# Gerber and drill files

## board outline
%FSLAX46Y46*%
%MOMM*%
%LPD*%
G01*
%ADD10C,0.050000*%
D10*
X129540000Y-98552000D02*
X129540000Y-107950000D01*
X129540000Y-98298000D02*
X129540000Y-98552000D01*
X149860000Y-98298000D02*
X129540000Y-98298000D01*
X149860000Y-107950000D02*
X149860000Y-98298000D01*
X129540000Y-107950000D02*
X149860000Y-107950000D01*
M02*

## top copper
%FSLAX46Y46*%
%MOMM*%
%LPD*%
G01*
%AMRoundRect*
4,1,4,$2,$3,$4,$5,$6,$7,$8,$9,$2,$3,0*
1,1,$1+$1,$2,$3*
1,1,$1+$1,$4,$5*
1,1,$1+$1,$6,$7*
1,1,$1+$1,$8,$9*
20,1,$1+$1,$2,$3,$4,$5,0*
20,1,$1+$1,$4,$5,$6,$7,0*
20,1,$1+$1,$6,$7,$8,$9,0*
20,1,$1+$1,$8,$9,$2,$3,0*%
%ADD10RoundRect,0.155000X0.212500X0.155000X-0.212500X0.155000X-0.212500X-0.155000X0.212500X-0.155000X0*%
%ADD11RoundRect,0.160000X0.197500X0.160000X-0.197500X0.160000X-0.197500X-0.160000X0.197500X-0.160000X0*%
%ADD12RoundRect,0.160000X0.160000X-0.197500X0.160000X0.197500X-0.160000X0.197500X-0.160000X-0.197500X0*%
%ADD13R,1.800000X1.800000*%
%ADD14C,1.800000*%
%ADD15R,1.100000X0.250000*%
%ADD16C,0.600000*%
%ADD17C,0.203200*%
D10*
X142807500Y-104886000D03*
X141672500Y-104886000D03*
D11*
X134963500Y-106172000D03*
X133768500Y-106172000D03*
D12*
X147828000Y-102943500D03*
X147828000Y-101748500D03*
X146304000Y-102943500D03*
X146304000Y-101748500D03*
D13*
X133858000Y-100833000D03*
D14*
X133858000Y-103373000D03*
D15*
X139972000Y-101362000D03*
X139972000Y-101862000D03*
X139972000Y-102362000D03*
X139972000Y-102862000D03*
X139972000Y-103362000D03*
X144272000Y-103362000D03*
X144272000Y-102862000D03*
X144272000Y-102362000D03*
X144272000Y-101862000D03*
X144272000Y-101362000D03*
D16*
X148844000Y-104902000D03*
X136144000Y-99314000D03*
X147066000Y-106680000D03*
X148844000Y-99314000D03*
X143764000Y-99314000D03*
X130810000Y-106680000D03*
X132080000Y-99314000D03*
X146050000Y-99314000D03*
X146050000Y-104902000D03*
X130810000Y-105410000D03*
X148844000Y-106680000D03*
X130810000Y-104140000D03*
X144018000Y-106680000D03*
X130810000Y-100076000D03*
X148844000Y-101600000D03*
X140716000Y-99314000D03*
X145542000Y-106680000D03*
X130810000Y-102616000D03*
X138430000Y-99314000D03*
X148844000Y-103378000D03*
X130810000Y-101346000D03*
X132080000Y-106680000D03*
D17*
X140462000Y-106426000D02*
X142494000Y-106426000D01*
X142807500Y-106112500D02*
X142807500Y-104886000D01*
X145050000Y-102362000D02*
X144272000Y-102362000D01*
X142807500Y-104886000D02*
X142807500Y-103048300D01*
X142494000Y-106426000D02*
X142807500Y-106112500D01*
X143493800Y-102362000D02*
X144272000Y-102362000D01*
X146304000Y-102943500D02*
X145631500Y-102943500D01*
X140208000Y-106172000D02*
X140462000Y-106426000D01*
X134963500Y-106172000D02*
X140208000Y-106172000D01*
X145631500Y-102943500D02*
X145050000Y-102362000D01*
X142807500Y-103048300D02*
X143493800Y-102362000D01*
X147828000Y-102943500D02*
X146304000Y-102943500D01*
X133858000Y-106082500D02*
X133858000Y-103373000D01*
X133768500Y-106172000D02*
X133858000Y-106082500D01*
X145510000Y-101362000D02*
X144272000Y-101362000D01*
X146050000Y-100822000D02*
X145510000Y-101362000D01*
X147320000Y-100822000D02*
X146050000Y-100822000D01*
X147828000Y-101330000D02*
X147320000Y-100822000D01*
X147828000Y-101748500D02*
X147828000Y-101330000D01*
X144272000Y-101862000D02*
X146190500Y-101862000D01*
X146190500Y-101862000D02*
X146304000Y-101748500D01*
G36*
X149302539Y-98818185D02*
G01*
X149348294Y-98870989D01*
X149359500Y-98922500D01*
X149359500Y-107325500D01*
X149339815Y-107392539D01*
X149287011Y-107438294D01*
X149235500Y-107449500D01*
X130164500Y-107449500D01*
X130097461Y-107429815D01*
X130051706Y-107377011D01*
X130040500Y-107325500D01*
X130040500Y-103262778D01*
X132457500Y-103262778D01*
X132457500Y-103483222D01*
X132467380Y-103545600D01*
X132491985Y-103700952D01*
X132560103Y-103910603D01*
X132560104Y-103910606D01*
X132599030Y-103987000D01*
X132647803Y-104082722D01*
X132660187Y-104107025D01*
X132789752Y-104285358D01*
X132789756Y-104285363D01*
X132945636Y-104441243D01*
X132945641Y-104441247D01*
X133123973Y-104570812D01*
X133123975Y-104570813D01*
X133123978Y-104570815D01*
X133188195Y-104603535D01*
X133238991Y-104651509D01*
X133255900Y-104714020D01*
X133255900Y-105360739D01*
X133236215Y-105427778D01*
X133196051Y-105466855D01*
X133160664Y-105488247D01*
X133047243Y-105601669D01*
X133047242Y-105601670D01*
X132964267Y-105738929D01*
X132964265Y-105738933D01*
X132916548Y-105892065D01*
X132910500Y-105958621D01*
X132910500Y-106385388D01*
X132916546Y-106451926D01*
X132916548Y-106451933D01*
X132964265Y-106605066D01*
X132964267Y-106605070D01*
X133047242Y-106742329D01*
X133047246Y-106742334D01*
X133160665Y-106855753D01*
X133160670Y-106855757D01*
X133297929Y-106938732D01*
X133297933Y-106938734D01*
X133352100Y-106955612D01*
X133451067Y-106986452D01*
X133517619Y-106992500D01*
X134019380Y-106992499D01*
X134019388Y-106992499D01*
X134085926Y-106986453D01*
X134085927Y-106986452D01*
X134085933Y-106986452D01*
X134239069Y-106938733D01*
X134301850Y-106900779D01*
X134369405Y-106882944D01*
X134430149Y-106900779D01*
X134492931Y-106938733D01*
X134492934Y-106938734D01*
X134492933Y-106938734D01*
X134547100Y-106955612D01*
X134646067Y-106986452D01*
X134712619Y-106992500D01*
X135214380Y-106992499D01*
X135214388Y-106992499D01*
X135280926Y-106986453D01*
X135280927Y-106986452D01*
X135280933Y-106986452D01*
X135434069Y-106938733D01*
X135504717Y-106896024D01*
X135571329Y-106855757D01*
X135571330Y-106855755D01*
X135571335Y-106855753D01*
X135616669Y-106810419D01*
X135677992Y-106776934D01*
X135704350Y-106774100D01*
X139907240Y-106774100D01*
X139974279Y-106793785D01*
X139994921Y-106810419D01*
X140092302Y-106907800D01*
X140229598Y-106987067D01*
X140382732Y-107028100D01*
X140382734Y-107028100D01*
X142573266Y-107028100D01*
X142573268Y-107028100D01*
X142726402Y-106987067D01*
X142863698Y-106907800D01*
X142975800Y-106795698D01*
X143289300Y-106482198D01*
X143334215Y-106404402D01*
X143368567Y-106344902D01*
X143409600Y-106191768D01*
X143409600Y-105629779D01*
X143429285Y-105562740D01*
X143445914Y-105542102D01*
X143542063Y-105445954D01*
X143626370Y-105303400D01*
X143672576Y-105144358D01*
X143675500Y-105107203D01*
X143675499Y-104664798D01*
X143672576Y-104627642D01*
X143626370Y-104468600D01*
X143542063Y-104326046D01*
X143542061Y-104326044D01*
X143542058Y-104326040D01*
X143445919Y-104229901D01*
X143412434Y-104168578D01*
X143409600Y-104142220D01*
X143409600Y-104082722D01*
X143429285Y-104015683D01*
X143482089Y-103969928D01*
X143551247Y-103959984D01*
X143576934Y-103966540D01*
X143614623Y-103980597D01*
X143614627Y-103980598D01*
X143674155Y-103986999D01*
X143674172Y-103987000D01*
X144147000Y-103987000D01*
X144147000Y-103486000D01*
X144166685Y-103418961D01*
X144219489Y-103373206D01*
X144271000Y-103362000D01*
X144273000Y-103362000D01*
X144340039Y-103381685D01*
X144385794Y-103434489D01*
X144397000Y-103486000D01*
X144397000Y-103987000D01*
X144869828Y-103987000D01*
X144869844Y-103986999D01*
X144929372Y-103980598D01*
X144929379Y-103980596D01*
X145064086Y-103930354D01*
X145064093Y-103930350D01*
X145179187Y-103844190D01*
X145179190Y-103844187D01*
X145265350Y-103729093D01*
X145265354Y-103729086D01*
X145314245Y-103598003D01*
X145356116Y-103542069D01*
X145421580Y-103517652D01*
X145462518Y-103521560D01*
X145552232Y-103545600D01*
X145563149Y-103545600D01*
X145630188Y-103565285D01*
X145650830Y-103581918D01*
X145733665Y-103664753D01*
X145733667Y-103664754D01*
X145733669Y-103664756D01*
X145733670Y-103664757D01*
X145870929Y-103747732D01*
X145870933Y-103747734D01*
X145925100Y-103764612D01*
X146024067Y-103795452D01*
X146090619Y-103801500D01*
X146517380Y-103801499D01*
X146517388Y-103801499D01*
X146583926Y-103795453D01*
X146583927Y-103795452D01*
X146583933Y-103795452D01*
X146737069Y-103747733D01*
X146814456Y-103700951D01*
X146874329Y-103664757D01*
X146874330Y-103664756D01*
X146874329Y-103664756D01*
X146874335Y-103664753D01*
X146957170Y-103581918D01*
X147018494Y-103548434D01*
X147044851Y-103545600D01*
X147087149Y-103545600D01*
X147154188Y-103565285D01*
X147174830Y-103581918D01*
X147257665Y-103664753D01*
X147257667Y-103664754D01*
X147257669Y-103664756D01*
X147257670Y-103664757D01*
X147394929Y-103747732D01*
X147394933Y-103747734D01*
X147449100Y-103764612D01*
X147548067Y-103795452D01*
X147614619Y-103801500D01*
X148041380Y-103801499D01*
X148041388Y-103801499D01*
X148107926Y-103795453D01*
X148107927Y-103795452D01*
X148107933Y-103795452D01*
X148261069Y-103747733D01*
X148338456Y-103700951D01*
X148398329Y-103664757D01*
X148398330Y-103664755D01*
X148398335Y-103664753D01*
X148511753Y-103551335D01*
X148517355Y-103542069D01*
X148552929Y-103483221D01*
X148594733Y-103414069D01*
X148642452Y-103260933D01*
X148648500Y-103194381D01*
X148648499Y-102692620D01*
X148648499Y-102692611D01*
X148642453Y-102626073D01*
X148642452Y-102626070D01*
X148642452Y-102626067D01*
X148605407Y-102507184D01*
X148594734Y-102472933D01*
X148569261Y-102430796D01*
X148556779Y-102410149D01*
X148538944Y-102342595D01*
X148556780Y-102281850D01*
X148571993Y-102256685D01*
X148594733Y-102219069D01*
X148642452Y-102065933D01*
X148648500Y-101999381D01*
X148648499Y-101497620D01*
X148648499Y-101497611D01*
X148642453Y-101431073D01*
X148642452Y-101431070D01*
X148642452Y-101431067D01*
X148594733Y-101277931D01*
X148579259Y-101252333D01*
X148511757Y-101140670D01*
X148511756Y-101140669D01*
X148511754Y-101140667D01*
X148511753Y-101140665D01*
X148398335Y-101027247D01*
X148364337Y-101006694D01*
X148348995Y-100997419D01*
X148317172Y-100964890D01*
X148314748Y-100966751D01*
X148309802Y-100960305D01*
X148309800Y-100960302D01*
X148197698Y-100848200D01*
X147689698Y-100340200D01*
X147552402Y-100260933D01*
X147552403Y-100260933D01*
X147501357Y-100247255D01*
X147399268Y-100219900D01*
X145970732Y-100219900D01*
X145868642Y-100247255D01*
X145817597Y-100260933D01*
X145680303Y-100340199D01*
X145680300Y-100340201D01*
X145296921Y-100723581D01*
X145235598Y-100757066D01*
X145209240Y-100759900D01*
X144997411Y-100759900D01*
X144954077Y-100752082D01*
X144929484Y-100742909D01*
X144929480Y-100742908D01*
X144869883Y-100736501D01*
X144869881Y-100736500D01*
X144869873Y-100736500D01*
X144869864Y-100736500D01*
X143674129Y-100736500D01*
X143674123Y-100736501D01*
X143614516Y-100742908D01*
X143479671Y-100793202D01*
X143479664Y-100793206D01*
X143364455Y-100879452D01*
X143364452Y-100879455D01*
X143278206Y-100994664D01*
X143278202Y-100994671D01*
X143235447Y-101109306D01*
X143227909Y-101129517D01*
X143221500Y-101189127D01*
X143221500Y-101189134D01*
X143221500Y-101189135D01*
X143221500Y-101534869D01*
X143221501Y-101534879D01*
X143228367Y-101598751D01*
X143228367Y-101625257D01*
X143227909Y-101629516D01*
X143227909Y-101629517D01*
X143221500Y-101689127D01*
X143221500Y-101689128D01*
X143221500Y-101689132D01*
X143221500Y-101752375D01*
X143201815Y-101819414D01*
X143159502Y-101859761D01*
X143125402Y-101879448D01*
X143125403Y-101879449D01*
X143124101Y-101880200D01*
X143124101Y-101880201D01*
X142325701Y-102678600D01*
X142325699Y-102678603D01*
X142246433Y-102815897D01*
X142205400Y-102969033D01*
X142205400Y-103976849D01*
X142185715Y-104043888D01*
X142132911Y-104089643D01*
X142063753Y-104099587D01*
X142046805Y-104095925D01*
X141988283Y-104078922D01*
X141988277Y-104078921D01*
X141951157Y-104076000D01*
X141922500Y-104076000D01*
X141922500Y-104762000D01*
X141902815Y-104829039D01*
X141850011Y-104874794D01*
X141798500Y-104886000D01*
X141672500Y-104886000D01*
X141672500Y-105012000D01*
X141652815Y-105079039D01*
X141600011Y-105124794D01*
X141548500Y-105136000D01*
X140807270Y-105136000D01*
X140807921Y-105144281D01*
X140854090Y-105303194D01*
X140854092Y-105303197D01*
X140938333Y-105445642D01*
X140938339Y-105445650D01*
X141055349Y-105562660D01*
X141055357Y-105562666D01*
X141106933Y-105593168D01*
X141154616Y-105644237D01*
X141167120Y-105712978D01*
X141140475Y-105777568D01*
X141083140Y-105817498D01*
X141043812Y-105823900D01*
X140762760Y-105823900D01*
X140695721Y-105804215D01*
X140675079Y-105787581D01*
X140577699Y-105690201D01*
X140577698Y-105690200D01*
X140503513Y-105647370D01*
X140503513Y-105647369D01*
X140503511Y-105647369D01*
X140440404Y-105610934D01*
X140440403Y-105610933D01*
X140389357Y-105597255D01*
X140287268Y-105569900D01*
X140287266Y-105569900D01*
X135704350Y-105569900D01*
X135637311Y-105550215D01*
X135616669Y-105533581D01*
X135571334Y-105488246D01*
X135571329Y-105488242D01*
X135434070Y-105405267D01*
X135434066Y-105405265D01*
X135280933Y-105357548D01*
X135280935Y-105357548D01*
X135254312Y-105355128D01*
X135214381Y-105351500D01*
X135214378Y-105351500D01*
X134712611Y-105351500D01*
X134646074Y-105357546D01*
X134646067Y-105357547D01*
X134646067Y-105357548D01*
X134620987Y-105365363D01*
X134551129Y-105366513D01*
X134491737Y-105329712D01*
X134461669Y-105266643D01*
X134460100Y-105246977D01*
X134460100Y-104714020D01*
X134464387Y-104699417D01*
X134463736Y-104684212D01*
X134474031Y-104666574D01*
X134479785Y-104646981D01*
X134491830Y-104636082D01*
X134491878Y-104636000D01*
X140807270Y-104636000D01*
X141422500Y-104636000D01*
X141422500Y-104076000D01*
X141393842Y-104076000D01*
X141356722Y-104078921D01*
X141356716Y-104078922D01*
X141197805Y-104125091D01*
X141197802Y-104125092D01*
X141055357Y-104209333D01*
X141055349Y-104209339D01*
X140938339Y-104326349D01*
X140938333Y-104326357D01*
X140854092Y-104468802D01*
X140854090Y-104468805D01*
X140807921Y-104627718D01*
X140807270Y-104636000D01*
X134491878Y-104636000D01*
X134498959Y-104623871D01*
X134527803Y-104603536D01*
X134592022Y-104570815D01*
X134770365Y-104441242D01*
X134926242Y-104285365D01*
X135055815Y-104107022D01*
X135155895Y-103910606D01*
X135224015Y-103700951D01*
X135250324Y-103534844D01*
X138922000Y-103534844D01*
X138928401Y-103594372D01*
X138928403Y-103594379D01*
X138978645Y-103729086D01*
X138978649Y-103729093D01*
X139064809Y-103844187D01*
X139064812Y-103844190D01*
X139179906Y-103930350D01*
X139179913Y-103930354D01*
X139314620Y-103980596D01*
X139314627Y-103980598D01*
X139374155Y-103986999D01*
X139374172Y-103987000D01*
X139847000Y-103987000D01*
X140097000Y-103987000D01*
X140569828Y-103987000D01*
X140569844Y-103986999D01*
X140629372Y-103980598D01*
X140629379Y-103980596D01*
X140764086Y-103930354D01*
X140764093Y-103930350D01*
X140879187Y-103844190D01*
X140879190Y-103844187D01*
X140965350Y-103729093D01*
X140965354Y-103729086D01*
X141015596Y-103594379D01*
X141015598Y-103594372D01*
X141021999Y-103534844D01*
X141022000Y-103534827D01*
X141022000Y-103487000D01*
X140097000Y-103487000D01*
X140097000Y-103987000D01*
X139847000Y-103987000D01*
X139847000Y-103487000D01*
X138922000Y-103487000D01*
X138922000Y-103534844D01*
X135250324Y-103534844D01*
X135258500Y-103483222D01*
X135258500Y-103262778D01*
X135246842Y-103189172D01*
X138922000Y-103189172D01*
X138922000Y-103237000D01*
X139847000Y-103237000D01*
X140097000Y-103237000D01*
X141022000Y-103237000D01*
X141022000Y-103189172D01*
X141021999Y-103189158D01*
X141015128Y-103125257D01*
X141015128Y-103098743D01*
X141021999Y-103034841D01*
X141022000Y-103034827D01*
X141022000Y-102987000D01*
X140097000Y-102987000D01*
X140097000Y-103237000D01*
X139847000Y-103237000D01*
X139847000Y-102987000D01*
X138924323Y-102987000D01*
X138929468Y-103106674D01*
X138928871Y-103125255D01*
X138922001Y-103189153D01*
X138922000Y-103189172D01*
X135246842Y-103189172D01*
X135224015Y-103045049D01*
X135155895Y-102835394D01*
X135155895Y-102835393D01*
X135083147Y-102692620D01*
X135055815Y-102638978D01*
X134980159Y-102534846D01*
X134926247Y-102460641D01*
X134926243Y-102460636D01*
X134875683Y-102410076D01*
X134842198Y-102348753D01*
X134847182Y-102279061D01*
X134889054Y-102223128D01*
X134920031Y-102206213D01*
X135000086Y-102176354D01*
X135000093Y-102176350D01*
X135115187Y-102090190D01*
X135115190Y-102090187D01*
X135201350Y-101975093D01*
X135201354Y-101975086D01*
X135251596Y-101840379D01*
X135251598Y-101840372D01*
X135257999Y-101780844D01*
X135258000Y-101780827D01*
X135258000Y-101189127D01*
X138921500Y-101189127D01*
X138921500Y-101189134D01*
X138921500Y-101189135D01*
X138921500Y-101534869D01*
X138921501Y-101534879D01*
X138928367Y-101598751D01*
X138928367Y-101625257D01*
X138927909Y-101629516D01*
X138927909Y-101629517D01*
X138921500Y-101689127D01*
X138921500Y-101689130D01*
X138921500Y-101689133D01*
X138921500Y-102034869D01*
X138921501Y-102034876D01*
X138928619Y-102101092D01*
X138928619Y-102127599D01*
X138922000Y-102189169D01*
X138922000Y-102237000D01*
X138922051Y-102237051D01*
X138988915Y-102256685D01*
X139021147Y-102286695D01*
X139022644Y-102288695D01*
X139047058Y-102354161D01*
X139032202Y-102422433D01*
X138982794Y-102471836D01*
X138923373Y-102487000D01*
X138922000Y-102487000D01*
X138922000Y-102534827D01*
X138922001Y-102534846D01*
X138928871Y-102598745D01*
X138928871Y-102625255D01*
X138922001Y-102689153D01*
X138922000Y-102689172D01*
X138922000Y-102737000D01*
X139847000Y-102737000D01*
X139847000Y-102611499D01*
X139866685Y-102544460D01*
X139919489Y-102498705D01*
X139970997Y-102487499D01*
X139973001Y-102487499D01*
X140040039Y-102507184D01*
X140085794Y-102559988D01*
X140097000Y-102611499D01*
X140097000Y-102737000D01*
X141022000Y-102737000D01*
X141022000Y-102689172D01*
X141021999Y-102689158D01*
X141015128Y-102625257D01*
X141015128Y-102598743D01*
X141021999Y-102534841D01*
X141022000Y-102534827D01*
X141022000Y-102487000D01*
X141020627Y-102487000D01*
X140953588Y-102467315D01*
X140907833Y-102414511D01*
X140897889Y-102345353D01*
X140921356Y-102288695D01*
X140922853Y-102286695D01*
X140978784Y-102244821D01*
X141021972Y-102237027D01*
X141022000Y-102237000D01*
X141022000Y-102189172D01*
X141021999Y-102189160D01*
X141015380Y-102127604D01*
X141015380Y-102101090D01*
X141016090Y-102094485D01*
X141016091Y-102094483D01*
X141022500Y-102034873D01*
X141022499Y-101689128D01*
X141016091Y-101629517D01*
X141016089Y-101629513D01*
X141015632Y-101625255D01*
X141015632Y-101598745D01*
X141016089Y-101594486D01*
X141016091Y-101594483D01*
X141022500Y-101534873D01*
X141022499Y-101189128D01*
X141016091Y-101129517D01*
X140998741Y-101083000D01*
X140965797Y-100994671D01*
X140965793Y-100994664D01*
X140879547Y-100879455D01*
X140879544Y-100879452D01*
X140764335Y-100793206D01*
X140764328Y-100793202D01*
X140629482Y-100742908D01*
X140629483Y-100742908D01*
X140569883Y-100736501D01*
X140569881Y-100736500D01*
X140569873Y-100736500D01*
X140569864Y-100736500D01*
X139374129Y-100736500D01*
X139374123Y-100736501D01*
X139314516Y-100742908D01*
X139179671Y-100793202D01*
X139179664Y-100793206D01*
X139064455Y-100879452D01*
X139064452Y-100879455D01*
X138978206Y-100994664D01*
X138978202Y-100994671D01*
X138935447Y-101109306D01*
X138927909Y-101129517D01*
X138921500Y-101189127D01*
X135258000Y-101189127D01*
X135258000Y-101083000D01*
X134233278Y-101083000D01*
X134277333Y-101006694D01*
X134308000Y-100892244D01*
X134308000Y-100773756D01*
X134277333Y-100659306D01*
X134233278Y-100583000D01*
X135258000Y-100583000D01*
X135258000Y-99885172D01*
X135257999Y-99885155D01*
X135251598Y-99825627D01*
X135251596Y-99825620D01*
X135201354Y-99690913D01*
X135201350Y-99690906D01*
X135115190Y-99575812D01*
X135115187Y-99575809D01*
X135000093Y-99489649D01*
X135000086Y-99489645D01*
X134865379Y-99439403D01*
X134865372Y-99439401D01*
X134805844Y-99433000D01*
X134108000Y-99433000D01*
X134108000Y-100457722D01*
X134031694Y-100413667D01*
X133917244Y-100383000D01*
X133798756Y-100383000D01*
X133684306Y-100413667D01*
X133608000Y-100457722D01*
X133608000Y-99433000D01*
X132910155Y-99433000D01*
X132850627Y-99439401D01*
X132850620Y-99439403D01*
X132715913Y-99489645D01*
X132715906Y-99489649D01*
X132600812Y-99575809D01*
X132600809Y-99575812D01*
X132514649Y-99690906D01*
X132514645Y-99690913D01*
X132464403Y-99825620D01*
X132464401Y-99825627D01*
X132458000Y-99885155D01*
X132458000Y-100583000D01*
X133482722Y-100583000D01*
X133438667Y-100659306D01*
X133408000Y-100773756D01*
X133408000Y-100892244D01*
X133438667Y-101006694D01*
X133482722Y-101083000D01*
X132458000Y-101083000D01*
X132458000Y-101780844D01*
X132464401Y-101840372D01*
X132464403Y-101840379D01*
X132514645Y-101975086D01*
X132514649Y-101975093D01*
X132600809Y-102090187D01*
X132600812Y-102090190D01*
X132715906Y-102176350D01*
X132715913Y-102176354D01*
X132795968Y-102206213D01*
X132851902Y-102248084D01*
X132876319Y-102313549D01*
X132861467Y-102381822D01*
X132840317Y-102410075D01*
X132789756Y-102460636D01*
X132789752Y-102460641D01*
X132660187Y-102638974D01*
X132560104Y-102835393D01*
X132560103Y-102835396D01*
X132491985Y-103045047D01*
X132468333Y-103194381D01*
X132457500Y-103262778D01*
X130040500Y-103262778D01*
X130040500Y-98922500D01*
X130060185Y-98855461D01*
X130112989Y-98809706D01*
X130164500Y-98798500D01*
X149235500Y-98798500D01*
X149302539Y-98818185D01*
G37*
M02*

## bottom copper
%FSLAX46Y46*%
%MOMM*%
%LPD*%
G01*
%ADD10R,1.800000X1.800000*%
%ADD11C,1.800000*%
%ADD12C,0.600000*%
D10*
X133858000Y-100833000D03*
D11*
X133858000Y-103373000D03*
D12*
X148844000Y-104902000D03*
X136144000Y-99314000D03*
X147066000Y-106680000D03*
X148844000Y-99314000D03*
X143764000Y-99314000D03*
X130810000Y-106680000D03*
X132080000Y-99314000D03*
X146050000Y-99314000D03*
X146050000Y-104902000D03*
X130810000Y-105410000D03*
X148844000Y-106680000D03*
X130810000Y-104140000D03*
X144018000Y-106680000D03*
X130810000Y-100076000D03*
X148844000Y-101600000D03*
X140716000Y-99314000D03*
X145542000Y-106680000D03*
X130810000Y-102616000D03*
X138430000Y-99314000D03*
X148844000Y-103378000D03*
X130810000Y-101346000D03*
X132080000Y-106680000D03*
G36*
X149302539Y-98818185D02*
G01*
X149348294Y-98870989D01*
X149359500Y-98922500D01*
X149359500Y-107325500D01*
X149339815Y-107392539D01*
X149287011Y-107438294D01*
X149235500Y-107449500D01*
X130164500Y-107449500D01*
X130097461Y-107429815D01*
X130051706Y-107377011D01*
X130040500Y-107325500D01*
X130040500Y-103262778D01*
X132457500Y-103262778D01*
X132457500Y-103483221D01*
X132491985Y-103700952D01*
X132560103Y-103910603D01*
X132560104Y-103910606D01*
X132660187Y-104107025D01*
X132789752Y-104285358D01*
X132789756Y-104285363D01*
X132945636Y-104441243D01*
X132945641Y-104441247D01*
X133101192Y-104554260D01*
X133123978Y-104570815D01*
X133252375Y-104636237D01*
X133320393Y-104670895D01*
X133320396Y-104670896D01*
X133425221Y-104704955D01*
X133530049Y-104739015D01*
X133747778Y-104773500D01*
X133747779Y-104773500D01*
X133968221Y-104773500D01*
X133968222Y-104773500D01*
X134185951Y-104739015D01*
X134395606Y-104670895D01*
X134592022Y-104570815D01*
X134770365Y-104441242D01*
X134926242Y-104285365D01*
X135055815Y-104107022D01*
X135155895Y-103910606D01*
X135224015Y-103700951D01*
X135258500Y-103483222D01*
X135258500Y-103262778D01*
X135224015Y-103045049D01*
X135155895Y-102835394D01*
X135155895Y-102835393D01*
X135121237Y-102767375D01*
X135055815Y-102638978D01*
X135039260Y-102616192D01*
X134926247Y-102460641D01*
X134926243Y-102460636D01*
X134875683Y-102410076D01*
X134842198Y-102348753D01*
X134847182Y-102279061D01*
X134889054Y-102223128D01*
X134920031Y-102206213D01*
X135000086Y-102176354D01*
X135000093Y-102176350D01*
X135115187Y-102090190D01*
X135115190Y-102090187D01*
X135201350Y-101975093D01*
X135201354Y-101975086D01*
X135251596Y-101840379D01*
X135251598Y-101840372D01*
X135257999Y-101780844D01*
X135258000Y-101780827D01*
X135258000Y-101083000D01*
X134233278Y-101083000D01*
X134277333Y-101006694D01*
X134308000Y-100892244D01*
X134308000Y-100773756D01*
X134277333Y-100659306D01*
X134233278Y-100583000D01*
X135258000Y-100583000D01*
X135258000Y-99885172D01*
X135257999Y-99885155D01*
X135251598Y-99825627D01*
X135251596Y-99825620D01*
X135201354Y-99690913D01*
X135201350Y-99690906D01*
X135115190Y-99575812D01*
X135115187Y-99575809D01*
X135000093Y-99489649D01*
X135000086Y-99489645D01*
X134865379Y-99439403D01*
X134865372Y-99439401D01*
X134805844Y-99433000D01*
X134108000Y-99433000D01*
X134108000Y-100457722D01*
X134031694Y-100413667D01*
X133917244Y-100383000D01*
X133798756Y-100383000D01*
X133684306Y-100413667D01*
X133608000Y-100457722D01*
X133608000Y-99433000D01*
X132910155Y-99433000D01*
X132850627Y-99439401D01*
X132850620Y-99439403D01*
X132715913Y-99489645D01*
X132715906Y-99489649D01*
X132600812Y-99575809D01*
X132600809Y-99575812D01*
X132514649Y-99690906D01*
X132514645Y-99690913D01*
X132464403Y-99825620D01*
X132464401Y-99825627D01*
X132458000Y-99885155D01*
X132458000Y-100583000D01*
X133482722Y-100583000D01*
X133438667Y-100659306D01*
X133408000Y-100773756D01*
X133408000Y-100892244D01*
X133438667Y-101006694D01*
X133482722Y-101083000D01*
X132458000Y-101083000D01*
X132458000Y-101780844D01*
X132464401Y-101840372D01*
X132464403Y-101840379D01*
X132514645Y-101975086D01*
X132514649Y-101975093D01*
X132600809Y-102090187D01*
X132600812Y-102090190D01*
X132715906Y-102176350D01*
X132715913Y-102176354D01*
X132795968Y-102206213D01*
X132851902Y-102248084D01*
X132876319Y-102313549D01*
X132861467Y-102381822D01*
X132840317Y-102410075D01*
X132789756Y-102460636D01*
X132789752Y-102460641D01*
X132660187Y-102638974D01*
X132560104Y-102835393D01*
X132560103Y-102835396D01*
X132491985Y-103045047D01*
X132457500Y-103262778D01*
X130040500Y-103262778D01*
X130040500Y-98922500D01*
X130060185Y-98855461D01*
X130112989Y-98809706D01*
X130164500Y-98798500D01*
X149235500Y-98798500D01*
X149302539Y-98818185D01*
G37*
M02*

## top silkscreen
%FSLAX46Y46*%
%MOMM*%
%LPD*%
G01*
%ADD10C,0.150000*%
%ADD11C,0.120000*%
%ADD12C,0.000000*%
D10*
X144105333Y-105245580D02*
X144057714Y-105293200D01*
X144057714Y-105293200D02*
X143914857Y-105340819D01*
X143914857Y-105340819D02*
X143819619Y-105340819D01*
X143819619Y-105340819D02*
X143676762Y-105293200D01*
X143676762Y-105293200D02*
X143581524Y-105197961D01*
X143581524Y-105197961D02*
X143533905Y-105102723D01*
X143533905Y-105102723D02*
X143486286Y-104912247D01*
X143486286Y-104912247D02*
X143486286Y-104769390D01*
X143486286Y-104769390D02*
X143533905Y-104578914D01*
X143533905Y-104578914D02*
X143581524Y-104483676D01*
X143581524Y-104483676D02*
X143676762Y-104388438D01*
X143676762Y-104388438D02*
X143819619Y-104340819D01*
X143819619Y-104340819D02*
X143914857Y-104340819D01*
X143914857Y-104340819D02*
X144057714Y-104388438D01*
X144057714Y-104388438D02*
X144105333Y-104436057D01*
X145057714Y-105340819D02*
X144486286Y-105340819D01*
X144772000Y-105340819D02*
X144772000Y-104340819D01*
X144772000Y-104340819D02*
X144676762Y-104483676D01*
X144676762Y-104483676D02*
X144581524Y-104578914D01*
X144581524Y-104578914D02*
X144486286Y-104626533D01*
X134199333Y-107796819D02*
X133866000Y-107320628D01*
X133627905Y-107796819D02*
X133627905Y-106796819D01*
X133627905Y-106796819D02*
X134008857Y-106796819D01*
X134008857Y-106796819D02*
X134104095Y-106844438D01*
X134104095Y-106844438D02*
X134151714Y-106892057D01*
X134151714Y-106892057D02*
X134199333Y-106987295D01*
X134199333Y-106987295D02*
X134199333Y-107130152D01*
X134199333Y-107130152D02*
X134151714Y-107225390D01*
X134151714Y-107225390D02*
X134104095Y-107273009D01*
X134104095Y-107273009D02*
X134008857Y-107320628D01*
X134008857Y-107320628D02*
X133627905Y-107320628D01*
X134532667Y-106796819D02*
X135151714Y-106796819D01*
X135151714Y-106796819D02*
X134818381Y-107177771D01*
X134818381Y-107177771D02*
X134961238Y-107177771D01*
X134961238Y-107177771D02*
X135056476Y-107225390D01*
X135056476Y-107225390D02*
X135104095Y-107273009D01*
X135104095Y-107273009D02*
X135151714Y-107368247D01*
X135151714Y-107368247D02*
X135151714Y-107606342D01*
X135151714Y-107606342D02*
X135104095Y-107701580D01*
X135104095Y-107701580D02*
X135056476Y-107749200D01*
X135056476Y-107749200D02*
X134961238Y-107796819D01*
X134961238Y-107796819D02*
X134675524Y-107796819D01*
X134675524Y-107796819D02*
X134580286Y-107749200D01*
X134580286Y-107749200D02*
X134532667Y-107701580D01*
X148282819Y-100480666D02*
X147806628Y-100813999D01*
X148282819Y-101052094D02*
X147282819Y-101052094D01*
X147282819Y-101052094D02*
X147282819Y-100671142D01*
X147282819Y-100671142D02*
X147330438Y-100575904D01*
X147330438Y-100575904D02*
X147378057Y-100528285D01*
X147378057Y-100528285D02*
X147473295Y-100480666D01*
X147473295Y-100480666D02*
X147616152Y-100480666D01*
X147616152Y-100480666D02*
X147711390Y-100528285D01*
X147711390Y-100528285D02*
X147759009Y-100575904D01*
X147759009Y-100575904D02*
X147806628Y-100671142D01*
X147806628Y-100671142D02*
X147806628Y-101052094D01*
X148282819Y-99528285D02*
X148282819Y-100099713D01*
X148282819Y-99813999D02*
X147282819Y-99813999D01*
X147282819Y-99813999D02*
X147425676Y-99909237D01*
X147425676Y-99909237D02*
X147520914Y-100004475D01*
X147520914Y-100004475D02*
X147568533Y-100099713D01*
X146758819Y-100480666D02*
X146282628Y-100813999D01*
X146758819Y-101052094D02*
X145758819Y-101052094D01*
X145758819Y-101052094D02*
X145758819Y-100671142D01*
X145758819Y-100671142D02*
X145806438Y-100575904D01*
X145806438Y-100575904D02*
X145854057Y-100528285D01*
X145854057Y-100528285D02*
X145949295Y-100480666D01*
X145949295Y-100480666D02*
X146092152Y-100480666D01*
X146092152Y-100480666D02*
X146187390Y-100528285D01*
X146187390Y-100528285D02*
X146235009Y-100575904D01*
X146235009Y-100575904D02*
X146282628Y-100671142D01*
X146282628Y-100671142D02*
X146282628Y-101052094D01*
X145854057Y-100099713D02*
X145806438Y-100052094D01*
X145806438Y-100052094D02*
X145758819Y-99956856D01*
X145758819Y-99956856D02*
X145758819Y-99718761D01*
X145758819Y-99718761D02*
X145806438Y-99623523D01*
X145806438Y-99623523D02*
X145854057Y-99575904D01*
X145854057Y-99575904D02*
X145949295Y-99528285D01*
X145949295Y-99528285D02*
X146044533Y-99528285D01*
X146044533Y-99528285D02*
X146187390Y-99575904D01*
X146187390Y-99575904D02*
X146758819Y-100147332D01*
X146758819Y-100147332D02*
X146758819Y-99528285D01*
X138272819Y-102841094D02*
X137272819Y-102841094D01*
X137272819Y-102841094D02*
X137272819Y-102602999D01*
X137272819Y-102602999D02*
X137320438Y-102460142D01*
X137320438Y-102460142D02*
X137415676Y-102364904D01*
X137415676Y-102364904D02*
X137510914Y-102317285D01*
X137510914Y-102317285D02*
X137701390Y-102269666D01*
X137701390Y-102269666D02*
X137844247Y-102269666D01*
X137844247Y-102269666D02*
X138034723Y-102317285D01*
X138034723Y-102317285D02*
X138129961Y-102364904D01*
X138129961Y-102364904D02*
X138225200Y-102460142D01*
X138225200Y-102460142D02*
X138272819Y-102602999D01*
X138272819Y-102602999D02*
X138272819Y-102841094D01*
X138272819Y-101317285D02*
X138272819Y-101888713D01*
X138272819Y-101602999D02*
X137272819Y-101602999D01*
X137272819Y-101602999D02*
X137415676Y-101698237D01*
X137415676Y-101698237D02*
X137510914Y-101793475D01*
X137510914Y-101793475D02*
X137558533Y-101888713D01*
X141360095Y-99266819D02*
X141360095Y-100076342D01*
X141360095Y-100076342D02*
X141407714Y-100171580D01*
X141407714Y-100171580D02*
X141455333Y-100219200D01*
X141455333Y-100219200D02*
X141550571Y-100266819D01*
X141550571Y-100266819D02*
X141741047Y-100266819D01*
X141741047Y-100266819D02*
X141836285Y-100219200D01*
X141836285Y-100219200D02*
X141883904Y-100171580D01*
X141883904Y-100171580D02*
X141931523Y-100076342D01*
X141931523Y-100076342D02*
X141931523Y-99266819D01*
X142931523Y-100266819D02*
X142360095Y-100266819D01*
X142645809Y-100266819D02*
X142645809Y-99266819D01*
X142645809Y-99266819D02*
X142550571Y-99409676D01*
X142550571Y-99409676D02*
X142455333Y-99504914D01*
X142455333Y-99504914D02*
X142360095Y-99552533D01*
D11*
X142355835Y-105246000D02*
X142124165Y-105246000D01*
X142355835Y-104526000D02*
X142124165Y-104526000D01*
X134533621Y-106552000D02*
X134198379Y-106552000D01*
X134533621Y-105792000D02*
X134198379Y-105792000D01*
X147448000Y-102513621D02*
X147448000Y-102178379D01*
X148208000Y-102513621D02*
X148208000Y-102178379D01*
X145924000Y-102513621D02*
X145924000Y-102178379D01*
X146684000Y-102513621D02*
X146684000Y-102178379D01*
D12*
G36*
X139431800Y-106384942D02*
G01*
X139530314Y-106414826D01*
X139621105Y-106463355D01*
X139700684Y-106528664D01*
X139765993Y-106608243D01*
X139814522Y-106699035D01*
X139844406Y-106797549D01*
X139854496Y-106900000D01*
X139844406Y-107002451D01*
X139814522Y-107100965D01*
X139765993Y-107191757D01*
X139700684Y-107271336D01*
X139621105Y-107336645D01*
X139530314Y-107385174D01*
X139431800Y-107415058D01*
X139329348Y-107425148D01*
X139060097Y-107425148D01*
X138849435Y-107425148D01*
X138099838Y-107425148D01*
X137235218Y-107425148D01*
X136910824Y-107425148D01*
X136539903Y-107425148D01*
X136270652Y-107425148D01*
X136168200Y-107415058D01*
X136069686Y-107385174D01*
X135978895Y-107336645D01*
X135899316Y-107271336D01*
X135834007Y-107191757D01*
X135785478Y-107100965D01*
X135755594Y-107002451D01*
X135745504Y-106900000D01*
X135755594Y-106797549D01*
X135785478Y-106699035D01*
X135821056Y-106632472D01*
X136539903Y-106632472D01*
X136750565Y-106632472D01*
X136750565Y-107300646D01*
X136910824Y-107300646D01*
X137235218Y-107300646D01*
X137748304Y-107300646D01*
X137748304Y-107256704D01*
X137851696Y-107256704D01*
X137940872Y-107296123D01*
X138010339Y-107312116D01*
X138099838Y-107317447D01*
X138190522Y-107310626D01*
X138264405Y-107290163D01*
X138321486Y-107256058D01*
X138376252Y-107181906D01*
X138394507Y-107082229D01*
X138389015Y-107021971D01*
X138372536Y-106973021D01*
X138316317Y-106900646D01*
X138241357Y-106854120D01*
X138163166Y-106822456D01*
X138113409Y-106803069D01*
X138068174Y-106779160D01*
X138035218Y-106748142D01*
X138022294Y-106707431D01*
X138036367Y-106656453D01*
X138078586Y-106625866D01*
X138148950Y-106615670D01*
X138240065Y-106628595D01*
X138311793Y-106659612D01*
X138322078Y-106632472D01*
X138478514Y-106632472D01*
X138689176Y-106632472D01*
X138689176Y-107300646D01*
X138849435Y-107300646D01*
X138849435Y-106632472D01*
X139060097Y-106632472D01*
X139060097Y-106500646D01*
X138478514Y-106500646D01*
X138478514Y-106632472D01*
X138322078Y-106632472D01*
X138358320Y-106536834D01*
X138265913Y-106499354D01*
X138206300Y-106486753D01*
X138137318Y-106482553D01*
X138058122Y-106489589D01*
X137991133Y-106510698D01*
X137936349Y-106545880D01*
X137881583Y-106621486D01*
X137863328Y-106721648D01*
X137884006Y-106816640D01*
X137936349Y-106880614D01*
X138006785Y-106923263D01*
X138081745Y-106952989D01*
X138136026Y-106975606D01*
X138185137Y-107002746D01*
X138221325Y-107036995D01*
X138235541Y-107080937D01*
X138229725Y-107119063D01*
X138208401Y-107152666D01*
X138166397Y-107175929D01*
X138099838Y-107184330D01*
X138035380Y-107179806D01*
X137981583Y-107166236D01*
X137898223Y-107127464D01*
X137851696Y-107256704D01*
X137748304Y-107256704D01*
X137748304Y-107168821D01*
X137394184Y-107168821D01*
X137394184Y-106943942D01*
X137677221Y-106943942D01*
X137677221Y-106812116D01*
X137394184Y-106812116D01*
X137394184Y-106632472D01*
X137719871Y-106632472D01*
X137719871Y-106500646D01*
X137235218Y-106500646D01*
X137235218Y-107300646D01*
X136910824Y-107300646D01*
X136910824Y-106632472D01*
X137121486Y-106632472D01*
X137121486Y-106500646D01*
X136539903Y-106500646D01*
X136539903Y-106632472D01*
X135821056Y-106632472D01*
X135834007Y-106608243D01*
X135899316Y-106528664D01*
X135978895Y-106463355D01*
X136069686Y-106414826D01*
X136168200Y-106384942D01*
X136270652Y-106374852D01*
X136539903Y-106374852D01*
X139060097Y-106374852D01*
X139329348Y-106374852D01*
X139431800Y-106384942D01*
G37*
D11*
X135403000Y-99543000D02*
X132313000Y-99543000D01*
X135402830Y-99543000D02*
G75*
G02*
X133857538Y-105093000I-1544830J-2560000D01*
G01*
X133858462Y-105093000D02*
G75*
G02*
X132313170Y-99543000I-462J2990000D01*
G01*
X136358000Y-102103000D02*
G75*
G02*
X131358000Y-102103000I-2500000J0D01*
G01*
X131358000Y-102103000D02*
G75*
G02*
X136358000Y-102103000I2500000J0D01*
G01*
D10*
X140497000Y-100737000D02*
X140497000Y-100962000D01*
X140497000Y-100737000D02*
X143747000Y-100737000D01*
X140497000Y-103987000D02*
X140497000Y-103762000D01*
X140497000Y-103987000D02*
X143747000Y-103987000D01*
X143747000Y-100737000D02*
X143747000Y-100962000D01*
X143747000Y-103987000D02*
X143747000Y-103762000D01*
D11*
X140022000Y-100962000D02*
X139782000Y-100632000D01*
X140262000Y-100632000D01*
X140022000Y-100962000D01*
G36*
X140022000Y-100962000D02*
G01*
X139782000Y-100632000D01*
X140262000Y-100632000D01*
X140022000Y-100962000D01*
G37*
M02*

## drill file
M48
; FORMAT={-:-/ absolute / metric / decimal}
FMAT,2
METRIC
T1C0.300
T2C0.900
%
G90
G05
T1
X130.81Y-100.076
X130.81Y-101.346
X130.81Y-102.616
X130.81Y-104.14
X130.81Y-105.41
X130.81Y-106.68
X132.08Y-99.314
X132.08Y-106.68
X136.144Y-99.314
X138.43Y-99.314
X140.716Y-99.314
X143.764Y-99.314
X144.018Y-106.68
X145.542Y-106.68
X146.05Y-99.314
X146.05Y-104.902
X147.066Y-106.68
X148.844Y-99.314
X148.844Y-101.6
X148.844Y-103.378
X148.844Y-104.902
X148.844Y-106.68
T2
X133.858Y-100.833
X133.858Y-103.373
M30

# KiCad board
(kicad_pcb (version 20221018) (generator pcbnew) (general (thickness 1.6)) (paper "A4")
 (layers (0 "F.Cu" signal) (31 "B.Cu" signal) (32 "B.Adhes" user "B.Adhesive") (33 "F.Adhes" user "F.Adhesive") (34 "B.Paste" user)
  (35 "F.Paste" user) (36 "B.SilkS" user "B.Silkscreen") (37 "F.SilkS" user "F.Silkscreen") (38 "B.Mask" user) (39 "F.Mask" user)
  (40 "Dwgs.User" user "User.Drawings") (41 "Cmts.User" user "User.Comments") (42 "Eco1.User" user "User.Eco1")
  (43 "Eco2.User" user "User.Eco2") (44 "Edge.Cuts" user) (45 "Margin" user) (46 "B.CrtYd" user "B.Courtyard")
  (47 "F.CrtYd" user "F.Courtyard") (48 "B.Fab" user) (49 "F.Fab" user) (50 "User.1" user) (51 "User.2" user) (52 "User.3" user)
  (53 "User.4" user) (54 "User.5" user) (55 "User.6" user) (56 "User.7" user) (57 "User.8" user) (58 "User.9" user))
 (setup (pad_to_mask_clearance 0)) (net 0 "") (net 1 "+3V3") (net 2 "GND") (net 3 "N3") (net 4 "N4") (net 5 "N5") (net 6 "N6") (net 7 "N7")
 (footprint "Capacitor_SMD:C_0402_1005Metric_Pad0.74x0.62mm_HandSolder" (layer "F.Cu") (at 142.24 104.886 180)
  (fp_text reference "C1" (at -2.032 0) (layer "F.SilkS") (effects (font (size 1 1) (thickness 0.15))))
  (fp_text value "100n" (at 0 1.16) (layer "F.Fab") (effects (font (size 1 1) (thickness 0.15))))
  (fp_line (start -0.115835 -0.36) (end 0.115835 -0.36) (stroke (width 0.12) (type solid)) (layer "F.SilkS"))
  (fp_line (start -0.115835 0.36) (end 0.115835 0.36) (stroke (width 0.12) (type solid)) (layer "F.SilkS"))
  (pad "1" smd roundrect (at -0.5675 0 180) (size 0.735 0.62) (layers "F.Cu" "F.Paste" "F.Mask") (roundrect_rratio 0.25) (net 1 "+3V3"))
  (pad "2" smd roundrect (at 0.5675 0 180) (size 0.735 0.62) (layers "F.Cu" "F.Paste" "F.Mask") (roundrect_rratio 0.25) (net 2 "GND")))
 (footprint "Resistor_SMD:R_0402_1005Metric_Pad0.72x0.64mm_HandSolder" (layer "F.Cu") (at 134.366 106.172 180)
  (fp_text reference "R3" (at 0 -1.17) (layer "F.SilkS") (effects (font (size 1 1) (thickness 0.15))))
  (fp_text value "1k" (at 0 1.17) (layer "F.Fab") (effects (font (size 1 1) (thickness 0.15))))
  (fp_line (start -0.167621 -0.38) (end 0.167621 -0.38) (stroke (width 0.12) (type solid)) (layer "F.SilkS"))
  (fp_line (start -0.167621 0.38) (end 0.167621 0.38) (stroke (width 0.12) (type solid)) (layer "F.SilkS"))
  (pad "1" smd roundrect (at -0.5975 0 180) (size 0.715 0.64) (layers "F.Cu" "F.Paste" "F.Mask") (roundrect_rratio 0.25) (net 1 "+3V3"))
  (pad "2" smd roundrect (at 0.5975 0 180) (size 0.715 0.64) (layers "F.Cu" "F.Paste" "F.Mask") (roundrect_rratio 0.25) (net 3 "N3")))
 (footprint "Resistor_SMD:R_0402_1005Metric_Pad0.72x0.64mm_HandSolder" (layer "F.Cu") (at 147.828 102.346 90)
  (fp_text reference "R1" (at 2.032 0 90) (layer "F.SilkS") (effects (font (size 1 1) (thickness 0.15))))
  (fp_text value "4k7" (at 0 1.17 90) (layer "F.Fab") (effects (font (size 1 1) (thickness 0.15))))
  (fp_line (start -0.167621 -0.38) (end 0.167621 -0.38) (stroke (width 0.12) (type solid)) (layer "F.SilkS"))
  (fp_line (start -0.167621 0.38) (end 0.167621 0.38) (stroke (width 0.12) (type solid)) (layer "F.SilkS"))
  (pad "1" smd roundrect (at -0.5975 0 90) (size 0.715 0.64) (layers "F.Cu" "F.Paste" "F.Mask") (roundrect_rratio 0.25) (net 1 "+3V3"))
  (pad "2" smd roundrect (at 0.5975 0 90) (size 0.715 0.64) (layers "F.Cu" "F.Paste" "F.Mask") (roundrect_rratio 0.25) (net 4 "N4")))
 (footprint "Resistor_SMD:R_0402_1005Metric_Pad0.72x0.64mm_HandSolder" (layer "F.Cu") (at 146.304 102.346 90)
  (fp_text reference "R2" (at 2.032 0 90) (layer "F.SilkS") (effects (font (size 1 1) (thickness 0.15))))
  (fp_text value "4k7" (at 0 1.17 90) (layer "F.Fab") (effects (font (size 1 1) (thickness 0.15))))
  (fp_line (start -0.167621 -0.38) (end 0.167621 -0.38) (stroke (width 0.12) (type solid)) (layer "F.SilkS"))
  (fp_line (start -0.167621 0.38) (end 0.167621 0.38) (stroke (width 0.12) (type solid)) (layer "F.SilkS"))
  (pad "1" smd roundrect (at -0.5975 0 90) (size 0.715 0.64) (layers "F.Cu" "F.Paste" "F.Mask") (roundrect_rratio 0.25) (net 1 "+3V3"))
  (pad "2" smd roundrect (at 0.5975 0 90) (size 0.715 0.64) (layers "F.Cu" "F.Paste" "F.Mask") (roundrect_rratio 0.25) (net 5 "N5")))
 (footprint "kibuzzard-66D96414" (layer "F.Cu") (at 137.8 106.9)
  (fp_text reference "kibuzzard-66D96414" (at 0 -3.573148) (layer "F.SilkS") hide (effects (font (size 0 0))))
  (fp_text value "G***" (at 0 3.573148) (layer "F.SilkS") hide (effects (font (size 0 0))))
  (fp_poly
   (pts (xy -1.260097 -0.525148) (xy -1.529348 -0.525148) (xy -1.6318 -0.515058) (xy -1.730314 -0.485174) (xy -1.821105 -0.436645)
    (xy -1.900684 -0.371336) (xy -1.965993 -0.291757) (xy -2.014522 -0.200965) (xy -2.044406 -0.102451) (xy -2.054496 0)
    (xy -2.044406 0.102451) (xy -2.014522 0.200965) (xy -1.965993 0.291757) (xy -1.900684 0.371336) (xy -1.821105 0.436645)
    (xy -1.730314 0.485174) (xy -1.6318 0.515058) (xy -1.529348 0.525148) (xy -1.260097 0.525148) (xy -0.889176 0.525148)
    (xy -0.889176 0.400646) (xy -1.049435 0.400646) (xy -1.049435 -0.267528) (xy -1.260097 -0.267528) (xy -1.260097 -0.399354)
    (xy -0.678514 -0.399354) (xy -0.678514 -0.267528) (xy -0.889176 -0.267528) (xy -0.889176 0.400646) (xy -0.889176 0.525148)
    (xy -0.564782 0.525148) (xy -0.564782 0.400646) (xy -0.564782 -0.399354) (xy -0.080129 -0.399354) (xy -0.080129 -0.267528)
    (xy -0.405816 -0.267528) (xy -0.405816 -0.087884) (xy -0.122779 -0.087884) (xy -0.122779 0.043942) (xy -0.405816 0.043942)
    (xy -0.405816 0.268821) (xy -0.051696 0.268821) (xy -0.051696 0.400646) (xy -0.564782 0.400646) (xy -0.564782 0.525148)
    (xy 0.299838 0.525148) (xy 0.299838 0.417447) (xy 0.210339 0.412116) (xy 0.140872 0.396123) (xy 0.051696 0.356704)
    (xy 0.098223 0.227464) (xy 0.181583 0.266236) (xy 0.23538 0.279806) (xy 0.299838 0.28433) (xy 0.366397 0.275929) (xy 0.408401 0.252666)
    (xy 0.429725 0.219063) (xy 0.435541 0.180937) (xy 0.421325 0.136995) (xy 0.385137 0.102746) (xy 0.336026 0.075606)
    (xy 0.281745 0.052989) (xy 0.206785 0.023263) (xy 0.136349 -0.019386) (xy 0.084006 -0.08336) (xy 0.063328 -0.178352)
    (xy 0.081583 -0.278514) (xy 0.136349 -0.35412) (xy 0.191133 -0.389302) (xy 0.258122 -0.410411) (xy 0.337318 -0.417447)
    (xy 0.4063 -0.413247) (xy 0.465913 -0.400646) (xy 0.55832 -0.363166) (xy 0.511793 -0.240388) (xy 0.440065 -0.271405)
    (xy 0.34895 -0.28433) (xy 0.278586 -0.274134) (xy 0.236367 -0.243547) (xy 0.222294 -0.192569) (xy 0.235218 -0.151858)
    (xy 0.268174 -0.12084) (xy 0.313409 -0.096931) (xy 0.363166 -0.077544) (xy 0.441357 -0.04588) (xy 0.516317 0.000646)
    (xy 0.572536 0.073021) (xy 0.589015 0.121971) (xy 0.594507 0.182229) (xy 0.576252 0.281906) (xy 0.521486 0.356058)
    (xy 0.464405 0.390163) (xy 0.390522 0.410626) (xy 0.299838 0.417447) (xy 0.299838 0.525148) (xy 1.049435 0.525148)
    (xy 1.049435 0.400646) (xy 0.889176 0.400646) (xy 0.889176 -0.267528) (xy 0.678514 -0.267528) (xy 0.678514 -0.399354)
    (xy 1.260097 -0.399354) (xy 1.260097 -0.267528) (xy 1.049435 -0.267528) (xy 1.049435 0.400646) (xy 1.049435 0.525148)
    (xy 1.260097 0.525148) (xy 1.529348 0.525148) (xy 1.6318 0.515058) (xy 1.730314 0.485174) (xy 1.821105 0.436645) (xy 1.900684 0.371336)
    (xy 1.965993 0.291757) (xy 2.014522 0.200965) (xy 2.044406 0.102451) (xy 2.054496 0) (xy 2.044406 -0.102451) (xy 2.014522 -0.200965)
    (xy 1.965993 -0.291757) (xy 1.900684 -0.371336) (xy 1.821105 -0.436645) (xy 1.730314 -0.485174) (xy 1.6318 -0.515058)
    (xy 1.529348 -0.525148) (xy 1.260097 -0.525148) (xy -1.260097 -0.525148))
   (stroke (width 0) (type solid)) (fill solid) (layer "F.SilkS")))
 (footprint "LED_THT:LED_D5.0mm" (layer "F.Cu") (at 133.858 100.833 -90)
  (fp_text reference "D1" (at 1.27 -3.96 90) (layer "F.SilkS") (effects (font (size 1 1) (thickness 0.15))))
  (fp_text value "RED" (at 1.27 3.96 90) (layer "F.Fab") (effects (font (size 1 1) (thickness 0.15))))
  (fp_line (start -1.29 -1.545) (end -1.29 1.545) (stroke (width 0.12) (type solid)) (layer "F.SilkS"))
  (fp_arc (start -1.29 -1.54483) (mid 2.072002 -2.880433) (end 4.26 0.000462) (stroke (width 0.12) (type solid)) (layer "F.SilkS"))
  (fp_arc (start 4.26 -0.000462) (mid 2.072002 2.880433) (end -1.29 1.54483) (stroke (width 0.12) (type solid)) (layer "F.SilkS"))
  (fp_circle (center 1.27 0) (end 3.77 0) (stroke (width 0.12) (type solid)) (fill none) (layer "F.SilkS"))
  (pad "1" thru_hole rect (at 0 0 270) (size 1.8 1.8) (drill 0.9) (layers "*.Cu" "*.Mask") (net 2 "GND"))
  (pad "2" thru_hole circle (at 2.54 0 270) (size 1.8 1.8) (drill 0.9) (layers "*.Cu" "*.Mask") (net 3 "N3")))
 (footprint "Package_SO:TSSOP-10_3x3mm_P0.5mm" (layer "F.Cu") (at 142.122 102.362)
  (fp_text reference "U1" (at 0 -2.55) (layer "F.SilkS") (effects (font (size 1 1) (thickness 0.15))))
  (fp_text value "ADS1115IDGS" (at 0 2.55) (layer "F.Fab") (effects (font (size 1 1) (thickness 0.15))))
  (fp_line (start -1.625 -1.625) (end -1.625 -1.4) (stroke (width 0.15) (type solid)) (layer "F.SilkS"))
  (fp_line (start -1.625 -1.625) (end 1.625 -1.625) (stroke (width 0.15) (type solid)) (layer "F.SilkS"))
  (fp_line (start -1.625 1.625) (end -1.625 1.4) (stroke (width 0.15) (type solid)) (layer "F.SilkS"))
  (fp_line (start -1.625 1.625) (end 1.625 1.625) (stroke (width 0.15) (type solid)) (layer "F.SilkS"))
  (fp_line (start 1.625 -1.625) (end 1.625 -1.4) (stroke (width 0.15) (type solid)) (layer "F.SilkS"))
  (fp_line (start 1.625 1.625) (end 1.625 1.4) (stroke (width 0.15) (type solid)) (layer "F.SilkS"))
  (fp_poly
   (pts (xy -2.1 -1.4) (xy -2.34 -1.73) (xy -1.86 -1.73) (xy -2.1 -1.4)) (stroke (width 0.12) (type solid)) (fill solid) (layer "F.SilkS"))
  (pad "1" smd rect (at -2.15 -1) (size 1.1 0.25) (layers "F.Cu" "F.Paste" "F.Mask") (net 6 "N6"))
  (pad "2" smd rect (at -2.15 -0.5) (size 1.1 0.25) (layers "F.Cu" "F.Paste" "F.Mask") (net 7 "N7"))
  (pad "3" smd rect (at -2.15 0) (size 1.1 0.25) (layers "F.Cu" "F.Paste" "F.Mask") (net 2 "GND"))
  (pad "4" smd rect (at -2.15 0.5) (size 1.1 0.25) (layers "F.Cu" "F.Paste" "F.Mask") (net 2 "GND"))
  (pad "5" smd rect (at -2.15 1) (size 1.1 0.25) (layers "F.Cu" "F.Paste" "F.Mask") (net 2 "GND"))
  (pad "6" smd rect (at 2.15 1) (size 1.1 0.25) (layers "F.Cu" "F.Paste" "F.Mask") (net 2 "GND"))
  (pad "7" smd rect (at 2.15 0.5) (size 1.1 0.25) (layers "F.Cu" "F.Paste" "F.Mask") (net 2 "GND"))
  (pad "8" smd rect (at 2.15 0) (size 1.1 0.25) (layers "F.Cu" "F.Paste" "F.Mask") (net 1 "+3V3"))
  (pad "9" smd rect (at 2.15 -0.5) (size 1.1 0.25) (layers "F.Cu" "F.Paste" "F.Mask") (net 5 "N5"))
  (pad "10" smd rect (at 2.15 -1) (size 1.1 0.25) (layers "F.Cu" "F.Paste" "F.Mask") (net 4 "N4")))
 (gr_line (start 129.54 98.552) (end 129.54 107.95) (stroke (width 0.05) (type default)) (layer "Edge.Cuts"))
 (gr_line (start 129.54 98.298) (end 129.54 98.552) (stroke (width 0.05) (type default)) (layer "Edge.Cuts"))
 (gr_line (start 149.86 98.298) (end 129.54 98.298) (stroke (width 0.05) (type default)) (layer "Edge.Cuts"))
 (gr_line (start 149.86 107.95) (end 149.86 98.298) (stroke (width 0.05) (type default)) (layer "Edge.Cuts"))
 (gr_line (start 129.54 107.95) (end 149.86 107.95) (stroke (width 0.05) (type default)) (layer "Edge.Cuts"))
 (segment (start 140.462 106.426) (end 142.494 106.426) (width 0.2032) (layer "F.Cu") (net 1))
 (segment (start 142.8075 106.1125) (end 142.8075 104.886) (width 0.2032) (layer "F.Cu") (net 1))
 (segment (start 145.05 102.362) (end 144.272 102.362) (width 0.2032) (layer "F.Cu") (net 1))
 (segment (start 142.8075 104.886) (end 142.8075 103.0483) (width 0.2032) (layer "F.Cu") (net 1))
 (segment (start 142.494 106.426) (end 142.8075 106.1125) (width 0.2032) (layer "F.Cu") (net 1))
 (segment (start 143.4938 102.362) (end 144.272 102.362) (width 0.2032) (layer "F.Cu") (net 1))
 (segment (start 146.304 102.9435) (end 145.6315 102.9435) (width 0.2032) (layer "F.Cu") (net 1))
 (segment (start 140.208 106.172) (end 140.462 106.426) (width 0.2032) (layer "F.Cu") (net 1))
 (segment (start 134.9635 106.172) (end 140.208 106.172) (width 0.2032) (layer "F.Cu") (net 1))
 (segment (start 145.6315 102.9435) (end 145.05 102.362) (width 0.2032) (layer "F.Cu") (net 1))
 (segment (start 142.8075 103.0483) (end 143.4938 102.362) (width 0.2032) (layer "F.Cu") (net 1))
 (segment (start 147.828 102.9435) (end 146.304 102.9435) (width 0.2032) (layer "F.Cu") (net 1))
 (via (at 148.844 104.902) (size 0.6) (drill 0.3) (layers "F.Cu" "B.Cu") (free) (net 2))
 (via (at 136.144 99.314) (size 0.6) (drill 0.3) (layers "F.Cu" "B.Cu") (free) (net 2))
 (via (at 147.066 106.68) (size 0.6) (drill 0.3) (layers "F.Cu" "B.Cu") (free) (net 2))
 (via (at 148.844 99.314) (size 0.6) (drill 0.3) (layers "F.Cu" "B.Cu") (free) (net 2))
 (via (at 143.764 99.314) (size 0.6) (drill 0.3) (layers "F.Cu" "B.Cu") (free) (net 2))
 (via (at 130.81 106.68) (size 0.6) (drill 0.3) (layers "F.Cu" "B.Cu") (free) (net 2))
 (via (at 132.08 99.314) (size 0.6) (drill 0.3) (layers "F.Cu" "B.Cu") (free) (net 2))
 (via (at 146.05 99.314) (size 0.6) (drill 0.3) (layers "F.Cu" "B.Cu") (free) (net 2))
 (via (at 146.05 104.902) (size 0.6) (drill 0.3) (layers "F.Cu" "B.Cu") (free) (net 2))
 (via (at 130.81 105.41) (size 0.6) (drill 0.3) (layers "F.Cu" "B.Cu") (free) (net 2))
 (via (at 148.844 106.68) (size 0.6) (drill 0.3) (layers "F.Cu" "B.Cu") (free) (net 2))
 (via (at 130.81 104.14) (size 0.6) (drill 0.3) (layers "F.Cu" "B.Cu") (free) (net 2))
 (via (at 144.018 106.68) (size 0.6) (drill 0.3) (layers "F.Cu" "B.Cu") (free) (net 2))
 (via (at 130.81 100.076) (size 0.6) (drill 0.3) (layers "F.Cu" "B.Cu") (free) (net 2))
 (via (at 148.844 101.6) (size 0.6) (drill 0.3) (layers "F.Cu" "B.Cu") (free) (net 2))
 (via (at 140.716 99.314) (size 0.6) (drill 0.3) (layers "F.Cu" "B.Cu") (free) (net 2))
 (via (at 145.542 106.68) (size 0.6) (drill 0.3) (layers "F.Cu" "B.Cu") (free) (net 2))
 (via (at 130.81 102.616) (size 0.6) (drill 0.3) (layers "F.Cu" "B.Cu") (free) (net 2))
 (via (at 138.43 99.314) (size 0.6) (drill 0.3) (layers "F.Cu" "B.Cu") (free) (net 2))
 (via (at 148.844 103.378) (size 0.6) (drill 0.3) (layers "F.Cu" "B.Cu") (free) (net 2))
 (via (at 130.81 101.346) (size 0.6) (drill 0.3) (layers "F.Cu" "B.Cu") (free) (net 2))
 (via (at 132.08 106.68) (size 0.6) (drill 0.3) (layers "F.Cu" "B.Cu") (free) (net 2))
 (segment (start 133.858 106.0825) (end 133.858 103.373) (width 0.2032) (layer "F.Cu") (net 3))
 (segment (start 133.7685 106.172) (end 133.858 106.0825) (width 0.2032) (layer "F.Cu") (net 3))
 (segment (start 145.51 101.362) (end 144.272 101.362) (width 0.2032) (layer "F.Cu") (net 4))
 (segment (start 146.05 100.822) (end 145.51 101.362) (width 0.2032) (layer "F.Cu") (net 4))
 (segment (start 147.32 100.822) (end 146.05 100.822) (width 0.2032) (layer "F.Cu") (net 4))
 (segment (start 147.828 101.33) (end 147.32 100.822) (width 0.2032) (layer "F.Cu") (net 4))
 (segment (start 147.828 101.7485) (end 147.828 101.33) (width 0.2032) (layer "F.Cu") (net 4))
 (segment (start 144.272 101.862) (end 146.1905 101.862) (width 0.2032) (layer "F.Cu") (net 5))
 (segment (start 146.1905 101.862) (end 146.304 101.7485) (width 0.2032) (layer "F.Cu") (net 5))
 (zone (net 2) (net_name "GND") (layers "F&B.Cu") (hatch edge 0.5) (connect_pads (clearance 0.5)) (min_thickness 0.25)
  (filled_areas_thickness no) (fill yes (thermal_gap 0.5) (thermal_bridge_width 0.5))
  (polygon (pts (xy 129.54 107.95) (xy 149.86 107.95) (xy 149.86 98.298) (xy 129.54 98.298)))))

